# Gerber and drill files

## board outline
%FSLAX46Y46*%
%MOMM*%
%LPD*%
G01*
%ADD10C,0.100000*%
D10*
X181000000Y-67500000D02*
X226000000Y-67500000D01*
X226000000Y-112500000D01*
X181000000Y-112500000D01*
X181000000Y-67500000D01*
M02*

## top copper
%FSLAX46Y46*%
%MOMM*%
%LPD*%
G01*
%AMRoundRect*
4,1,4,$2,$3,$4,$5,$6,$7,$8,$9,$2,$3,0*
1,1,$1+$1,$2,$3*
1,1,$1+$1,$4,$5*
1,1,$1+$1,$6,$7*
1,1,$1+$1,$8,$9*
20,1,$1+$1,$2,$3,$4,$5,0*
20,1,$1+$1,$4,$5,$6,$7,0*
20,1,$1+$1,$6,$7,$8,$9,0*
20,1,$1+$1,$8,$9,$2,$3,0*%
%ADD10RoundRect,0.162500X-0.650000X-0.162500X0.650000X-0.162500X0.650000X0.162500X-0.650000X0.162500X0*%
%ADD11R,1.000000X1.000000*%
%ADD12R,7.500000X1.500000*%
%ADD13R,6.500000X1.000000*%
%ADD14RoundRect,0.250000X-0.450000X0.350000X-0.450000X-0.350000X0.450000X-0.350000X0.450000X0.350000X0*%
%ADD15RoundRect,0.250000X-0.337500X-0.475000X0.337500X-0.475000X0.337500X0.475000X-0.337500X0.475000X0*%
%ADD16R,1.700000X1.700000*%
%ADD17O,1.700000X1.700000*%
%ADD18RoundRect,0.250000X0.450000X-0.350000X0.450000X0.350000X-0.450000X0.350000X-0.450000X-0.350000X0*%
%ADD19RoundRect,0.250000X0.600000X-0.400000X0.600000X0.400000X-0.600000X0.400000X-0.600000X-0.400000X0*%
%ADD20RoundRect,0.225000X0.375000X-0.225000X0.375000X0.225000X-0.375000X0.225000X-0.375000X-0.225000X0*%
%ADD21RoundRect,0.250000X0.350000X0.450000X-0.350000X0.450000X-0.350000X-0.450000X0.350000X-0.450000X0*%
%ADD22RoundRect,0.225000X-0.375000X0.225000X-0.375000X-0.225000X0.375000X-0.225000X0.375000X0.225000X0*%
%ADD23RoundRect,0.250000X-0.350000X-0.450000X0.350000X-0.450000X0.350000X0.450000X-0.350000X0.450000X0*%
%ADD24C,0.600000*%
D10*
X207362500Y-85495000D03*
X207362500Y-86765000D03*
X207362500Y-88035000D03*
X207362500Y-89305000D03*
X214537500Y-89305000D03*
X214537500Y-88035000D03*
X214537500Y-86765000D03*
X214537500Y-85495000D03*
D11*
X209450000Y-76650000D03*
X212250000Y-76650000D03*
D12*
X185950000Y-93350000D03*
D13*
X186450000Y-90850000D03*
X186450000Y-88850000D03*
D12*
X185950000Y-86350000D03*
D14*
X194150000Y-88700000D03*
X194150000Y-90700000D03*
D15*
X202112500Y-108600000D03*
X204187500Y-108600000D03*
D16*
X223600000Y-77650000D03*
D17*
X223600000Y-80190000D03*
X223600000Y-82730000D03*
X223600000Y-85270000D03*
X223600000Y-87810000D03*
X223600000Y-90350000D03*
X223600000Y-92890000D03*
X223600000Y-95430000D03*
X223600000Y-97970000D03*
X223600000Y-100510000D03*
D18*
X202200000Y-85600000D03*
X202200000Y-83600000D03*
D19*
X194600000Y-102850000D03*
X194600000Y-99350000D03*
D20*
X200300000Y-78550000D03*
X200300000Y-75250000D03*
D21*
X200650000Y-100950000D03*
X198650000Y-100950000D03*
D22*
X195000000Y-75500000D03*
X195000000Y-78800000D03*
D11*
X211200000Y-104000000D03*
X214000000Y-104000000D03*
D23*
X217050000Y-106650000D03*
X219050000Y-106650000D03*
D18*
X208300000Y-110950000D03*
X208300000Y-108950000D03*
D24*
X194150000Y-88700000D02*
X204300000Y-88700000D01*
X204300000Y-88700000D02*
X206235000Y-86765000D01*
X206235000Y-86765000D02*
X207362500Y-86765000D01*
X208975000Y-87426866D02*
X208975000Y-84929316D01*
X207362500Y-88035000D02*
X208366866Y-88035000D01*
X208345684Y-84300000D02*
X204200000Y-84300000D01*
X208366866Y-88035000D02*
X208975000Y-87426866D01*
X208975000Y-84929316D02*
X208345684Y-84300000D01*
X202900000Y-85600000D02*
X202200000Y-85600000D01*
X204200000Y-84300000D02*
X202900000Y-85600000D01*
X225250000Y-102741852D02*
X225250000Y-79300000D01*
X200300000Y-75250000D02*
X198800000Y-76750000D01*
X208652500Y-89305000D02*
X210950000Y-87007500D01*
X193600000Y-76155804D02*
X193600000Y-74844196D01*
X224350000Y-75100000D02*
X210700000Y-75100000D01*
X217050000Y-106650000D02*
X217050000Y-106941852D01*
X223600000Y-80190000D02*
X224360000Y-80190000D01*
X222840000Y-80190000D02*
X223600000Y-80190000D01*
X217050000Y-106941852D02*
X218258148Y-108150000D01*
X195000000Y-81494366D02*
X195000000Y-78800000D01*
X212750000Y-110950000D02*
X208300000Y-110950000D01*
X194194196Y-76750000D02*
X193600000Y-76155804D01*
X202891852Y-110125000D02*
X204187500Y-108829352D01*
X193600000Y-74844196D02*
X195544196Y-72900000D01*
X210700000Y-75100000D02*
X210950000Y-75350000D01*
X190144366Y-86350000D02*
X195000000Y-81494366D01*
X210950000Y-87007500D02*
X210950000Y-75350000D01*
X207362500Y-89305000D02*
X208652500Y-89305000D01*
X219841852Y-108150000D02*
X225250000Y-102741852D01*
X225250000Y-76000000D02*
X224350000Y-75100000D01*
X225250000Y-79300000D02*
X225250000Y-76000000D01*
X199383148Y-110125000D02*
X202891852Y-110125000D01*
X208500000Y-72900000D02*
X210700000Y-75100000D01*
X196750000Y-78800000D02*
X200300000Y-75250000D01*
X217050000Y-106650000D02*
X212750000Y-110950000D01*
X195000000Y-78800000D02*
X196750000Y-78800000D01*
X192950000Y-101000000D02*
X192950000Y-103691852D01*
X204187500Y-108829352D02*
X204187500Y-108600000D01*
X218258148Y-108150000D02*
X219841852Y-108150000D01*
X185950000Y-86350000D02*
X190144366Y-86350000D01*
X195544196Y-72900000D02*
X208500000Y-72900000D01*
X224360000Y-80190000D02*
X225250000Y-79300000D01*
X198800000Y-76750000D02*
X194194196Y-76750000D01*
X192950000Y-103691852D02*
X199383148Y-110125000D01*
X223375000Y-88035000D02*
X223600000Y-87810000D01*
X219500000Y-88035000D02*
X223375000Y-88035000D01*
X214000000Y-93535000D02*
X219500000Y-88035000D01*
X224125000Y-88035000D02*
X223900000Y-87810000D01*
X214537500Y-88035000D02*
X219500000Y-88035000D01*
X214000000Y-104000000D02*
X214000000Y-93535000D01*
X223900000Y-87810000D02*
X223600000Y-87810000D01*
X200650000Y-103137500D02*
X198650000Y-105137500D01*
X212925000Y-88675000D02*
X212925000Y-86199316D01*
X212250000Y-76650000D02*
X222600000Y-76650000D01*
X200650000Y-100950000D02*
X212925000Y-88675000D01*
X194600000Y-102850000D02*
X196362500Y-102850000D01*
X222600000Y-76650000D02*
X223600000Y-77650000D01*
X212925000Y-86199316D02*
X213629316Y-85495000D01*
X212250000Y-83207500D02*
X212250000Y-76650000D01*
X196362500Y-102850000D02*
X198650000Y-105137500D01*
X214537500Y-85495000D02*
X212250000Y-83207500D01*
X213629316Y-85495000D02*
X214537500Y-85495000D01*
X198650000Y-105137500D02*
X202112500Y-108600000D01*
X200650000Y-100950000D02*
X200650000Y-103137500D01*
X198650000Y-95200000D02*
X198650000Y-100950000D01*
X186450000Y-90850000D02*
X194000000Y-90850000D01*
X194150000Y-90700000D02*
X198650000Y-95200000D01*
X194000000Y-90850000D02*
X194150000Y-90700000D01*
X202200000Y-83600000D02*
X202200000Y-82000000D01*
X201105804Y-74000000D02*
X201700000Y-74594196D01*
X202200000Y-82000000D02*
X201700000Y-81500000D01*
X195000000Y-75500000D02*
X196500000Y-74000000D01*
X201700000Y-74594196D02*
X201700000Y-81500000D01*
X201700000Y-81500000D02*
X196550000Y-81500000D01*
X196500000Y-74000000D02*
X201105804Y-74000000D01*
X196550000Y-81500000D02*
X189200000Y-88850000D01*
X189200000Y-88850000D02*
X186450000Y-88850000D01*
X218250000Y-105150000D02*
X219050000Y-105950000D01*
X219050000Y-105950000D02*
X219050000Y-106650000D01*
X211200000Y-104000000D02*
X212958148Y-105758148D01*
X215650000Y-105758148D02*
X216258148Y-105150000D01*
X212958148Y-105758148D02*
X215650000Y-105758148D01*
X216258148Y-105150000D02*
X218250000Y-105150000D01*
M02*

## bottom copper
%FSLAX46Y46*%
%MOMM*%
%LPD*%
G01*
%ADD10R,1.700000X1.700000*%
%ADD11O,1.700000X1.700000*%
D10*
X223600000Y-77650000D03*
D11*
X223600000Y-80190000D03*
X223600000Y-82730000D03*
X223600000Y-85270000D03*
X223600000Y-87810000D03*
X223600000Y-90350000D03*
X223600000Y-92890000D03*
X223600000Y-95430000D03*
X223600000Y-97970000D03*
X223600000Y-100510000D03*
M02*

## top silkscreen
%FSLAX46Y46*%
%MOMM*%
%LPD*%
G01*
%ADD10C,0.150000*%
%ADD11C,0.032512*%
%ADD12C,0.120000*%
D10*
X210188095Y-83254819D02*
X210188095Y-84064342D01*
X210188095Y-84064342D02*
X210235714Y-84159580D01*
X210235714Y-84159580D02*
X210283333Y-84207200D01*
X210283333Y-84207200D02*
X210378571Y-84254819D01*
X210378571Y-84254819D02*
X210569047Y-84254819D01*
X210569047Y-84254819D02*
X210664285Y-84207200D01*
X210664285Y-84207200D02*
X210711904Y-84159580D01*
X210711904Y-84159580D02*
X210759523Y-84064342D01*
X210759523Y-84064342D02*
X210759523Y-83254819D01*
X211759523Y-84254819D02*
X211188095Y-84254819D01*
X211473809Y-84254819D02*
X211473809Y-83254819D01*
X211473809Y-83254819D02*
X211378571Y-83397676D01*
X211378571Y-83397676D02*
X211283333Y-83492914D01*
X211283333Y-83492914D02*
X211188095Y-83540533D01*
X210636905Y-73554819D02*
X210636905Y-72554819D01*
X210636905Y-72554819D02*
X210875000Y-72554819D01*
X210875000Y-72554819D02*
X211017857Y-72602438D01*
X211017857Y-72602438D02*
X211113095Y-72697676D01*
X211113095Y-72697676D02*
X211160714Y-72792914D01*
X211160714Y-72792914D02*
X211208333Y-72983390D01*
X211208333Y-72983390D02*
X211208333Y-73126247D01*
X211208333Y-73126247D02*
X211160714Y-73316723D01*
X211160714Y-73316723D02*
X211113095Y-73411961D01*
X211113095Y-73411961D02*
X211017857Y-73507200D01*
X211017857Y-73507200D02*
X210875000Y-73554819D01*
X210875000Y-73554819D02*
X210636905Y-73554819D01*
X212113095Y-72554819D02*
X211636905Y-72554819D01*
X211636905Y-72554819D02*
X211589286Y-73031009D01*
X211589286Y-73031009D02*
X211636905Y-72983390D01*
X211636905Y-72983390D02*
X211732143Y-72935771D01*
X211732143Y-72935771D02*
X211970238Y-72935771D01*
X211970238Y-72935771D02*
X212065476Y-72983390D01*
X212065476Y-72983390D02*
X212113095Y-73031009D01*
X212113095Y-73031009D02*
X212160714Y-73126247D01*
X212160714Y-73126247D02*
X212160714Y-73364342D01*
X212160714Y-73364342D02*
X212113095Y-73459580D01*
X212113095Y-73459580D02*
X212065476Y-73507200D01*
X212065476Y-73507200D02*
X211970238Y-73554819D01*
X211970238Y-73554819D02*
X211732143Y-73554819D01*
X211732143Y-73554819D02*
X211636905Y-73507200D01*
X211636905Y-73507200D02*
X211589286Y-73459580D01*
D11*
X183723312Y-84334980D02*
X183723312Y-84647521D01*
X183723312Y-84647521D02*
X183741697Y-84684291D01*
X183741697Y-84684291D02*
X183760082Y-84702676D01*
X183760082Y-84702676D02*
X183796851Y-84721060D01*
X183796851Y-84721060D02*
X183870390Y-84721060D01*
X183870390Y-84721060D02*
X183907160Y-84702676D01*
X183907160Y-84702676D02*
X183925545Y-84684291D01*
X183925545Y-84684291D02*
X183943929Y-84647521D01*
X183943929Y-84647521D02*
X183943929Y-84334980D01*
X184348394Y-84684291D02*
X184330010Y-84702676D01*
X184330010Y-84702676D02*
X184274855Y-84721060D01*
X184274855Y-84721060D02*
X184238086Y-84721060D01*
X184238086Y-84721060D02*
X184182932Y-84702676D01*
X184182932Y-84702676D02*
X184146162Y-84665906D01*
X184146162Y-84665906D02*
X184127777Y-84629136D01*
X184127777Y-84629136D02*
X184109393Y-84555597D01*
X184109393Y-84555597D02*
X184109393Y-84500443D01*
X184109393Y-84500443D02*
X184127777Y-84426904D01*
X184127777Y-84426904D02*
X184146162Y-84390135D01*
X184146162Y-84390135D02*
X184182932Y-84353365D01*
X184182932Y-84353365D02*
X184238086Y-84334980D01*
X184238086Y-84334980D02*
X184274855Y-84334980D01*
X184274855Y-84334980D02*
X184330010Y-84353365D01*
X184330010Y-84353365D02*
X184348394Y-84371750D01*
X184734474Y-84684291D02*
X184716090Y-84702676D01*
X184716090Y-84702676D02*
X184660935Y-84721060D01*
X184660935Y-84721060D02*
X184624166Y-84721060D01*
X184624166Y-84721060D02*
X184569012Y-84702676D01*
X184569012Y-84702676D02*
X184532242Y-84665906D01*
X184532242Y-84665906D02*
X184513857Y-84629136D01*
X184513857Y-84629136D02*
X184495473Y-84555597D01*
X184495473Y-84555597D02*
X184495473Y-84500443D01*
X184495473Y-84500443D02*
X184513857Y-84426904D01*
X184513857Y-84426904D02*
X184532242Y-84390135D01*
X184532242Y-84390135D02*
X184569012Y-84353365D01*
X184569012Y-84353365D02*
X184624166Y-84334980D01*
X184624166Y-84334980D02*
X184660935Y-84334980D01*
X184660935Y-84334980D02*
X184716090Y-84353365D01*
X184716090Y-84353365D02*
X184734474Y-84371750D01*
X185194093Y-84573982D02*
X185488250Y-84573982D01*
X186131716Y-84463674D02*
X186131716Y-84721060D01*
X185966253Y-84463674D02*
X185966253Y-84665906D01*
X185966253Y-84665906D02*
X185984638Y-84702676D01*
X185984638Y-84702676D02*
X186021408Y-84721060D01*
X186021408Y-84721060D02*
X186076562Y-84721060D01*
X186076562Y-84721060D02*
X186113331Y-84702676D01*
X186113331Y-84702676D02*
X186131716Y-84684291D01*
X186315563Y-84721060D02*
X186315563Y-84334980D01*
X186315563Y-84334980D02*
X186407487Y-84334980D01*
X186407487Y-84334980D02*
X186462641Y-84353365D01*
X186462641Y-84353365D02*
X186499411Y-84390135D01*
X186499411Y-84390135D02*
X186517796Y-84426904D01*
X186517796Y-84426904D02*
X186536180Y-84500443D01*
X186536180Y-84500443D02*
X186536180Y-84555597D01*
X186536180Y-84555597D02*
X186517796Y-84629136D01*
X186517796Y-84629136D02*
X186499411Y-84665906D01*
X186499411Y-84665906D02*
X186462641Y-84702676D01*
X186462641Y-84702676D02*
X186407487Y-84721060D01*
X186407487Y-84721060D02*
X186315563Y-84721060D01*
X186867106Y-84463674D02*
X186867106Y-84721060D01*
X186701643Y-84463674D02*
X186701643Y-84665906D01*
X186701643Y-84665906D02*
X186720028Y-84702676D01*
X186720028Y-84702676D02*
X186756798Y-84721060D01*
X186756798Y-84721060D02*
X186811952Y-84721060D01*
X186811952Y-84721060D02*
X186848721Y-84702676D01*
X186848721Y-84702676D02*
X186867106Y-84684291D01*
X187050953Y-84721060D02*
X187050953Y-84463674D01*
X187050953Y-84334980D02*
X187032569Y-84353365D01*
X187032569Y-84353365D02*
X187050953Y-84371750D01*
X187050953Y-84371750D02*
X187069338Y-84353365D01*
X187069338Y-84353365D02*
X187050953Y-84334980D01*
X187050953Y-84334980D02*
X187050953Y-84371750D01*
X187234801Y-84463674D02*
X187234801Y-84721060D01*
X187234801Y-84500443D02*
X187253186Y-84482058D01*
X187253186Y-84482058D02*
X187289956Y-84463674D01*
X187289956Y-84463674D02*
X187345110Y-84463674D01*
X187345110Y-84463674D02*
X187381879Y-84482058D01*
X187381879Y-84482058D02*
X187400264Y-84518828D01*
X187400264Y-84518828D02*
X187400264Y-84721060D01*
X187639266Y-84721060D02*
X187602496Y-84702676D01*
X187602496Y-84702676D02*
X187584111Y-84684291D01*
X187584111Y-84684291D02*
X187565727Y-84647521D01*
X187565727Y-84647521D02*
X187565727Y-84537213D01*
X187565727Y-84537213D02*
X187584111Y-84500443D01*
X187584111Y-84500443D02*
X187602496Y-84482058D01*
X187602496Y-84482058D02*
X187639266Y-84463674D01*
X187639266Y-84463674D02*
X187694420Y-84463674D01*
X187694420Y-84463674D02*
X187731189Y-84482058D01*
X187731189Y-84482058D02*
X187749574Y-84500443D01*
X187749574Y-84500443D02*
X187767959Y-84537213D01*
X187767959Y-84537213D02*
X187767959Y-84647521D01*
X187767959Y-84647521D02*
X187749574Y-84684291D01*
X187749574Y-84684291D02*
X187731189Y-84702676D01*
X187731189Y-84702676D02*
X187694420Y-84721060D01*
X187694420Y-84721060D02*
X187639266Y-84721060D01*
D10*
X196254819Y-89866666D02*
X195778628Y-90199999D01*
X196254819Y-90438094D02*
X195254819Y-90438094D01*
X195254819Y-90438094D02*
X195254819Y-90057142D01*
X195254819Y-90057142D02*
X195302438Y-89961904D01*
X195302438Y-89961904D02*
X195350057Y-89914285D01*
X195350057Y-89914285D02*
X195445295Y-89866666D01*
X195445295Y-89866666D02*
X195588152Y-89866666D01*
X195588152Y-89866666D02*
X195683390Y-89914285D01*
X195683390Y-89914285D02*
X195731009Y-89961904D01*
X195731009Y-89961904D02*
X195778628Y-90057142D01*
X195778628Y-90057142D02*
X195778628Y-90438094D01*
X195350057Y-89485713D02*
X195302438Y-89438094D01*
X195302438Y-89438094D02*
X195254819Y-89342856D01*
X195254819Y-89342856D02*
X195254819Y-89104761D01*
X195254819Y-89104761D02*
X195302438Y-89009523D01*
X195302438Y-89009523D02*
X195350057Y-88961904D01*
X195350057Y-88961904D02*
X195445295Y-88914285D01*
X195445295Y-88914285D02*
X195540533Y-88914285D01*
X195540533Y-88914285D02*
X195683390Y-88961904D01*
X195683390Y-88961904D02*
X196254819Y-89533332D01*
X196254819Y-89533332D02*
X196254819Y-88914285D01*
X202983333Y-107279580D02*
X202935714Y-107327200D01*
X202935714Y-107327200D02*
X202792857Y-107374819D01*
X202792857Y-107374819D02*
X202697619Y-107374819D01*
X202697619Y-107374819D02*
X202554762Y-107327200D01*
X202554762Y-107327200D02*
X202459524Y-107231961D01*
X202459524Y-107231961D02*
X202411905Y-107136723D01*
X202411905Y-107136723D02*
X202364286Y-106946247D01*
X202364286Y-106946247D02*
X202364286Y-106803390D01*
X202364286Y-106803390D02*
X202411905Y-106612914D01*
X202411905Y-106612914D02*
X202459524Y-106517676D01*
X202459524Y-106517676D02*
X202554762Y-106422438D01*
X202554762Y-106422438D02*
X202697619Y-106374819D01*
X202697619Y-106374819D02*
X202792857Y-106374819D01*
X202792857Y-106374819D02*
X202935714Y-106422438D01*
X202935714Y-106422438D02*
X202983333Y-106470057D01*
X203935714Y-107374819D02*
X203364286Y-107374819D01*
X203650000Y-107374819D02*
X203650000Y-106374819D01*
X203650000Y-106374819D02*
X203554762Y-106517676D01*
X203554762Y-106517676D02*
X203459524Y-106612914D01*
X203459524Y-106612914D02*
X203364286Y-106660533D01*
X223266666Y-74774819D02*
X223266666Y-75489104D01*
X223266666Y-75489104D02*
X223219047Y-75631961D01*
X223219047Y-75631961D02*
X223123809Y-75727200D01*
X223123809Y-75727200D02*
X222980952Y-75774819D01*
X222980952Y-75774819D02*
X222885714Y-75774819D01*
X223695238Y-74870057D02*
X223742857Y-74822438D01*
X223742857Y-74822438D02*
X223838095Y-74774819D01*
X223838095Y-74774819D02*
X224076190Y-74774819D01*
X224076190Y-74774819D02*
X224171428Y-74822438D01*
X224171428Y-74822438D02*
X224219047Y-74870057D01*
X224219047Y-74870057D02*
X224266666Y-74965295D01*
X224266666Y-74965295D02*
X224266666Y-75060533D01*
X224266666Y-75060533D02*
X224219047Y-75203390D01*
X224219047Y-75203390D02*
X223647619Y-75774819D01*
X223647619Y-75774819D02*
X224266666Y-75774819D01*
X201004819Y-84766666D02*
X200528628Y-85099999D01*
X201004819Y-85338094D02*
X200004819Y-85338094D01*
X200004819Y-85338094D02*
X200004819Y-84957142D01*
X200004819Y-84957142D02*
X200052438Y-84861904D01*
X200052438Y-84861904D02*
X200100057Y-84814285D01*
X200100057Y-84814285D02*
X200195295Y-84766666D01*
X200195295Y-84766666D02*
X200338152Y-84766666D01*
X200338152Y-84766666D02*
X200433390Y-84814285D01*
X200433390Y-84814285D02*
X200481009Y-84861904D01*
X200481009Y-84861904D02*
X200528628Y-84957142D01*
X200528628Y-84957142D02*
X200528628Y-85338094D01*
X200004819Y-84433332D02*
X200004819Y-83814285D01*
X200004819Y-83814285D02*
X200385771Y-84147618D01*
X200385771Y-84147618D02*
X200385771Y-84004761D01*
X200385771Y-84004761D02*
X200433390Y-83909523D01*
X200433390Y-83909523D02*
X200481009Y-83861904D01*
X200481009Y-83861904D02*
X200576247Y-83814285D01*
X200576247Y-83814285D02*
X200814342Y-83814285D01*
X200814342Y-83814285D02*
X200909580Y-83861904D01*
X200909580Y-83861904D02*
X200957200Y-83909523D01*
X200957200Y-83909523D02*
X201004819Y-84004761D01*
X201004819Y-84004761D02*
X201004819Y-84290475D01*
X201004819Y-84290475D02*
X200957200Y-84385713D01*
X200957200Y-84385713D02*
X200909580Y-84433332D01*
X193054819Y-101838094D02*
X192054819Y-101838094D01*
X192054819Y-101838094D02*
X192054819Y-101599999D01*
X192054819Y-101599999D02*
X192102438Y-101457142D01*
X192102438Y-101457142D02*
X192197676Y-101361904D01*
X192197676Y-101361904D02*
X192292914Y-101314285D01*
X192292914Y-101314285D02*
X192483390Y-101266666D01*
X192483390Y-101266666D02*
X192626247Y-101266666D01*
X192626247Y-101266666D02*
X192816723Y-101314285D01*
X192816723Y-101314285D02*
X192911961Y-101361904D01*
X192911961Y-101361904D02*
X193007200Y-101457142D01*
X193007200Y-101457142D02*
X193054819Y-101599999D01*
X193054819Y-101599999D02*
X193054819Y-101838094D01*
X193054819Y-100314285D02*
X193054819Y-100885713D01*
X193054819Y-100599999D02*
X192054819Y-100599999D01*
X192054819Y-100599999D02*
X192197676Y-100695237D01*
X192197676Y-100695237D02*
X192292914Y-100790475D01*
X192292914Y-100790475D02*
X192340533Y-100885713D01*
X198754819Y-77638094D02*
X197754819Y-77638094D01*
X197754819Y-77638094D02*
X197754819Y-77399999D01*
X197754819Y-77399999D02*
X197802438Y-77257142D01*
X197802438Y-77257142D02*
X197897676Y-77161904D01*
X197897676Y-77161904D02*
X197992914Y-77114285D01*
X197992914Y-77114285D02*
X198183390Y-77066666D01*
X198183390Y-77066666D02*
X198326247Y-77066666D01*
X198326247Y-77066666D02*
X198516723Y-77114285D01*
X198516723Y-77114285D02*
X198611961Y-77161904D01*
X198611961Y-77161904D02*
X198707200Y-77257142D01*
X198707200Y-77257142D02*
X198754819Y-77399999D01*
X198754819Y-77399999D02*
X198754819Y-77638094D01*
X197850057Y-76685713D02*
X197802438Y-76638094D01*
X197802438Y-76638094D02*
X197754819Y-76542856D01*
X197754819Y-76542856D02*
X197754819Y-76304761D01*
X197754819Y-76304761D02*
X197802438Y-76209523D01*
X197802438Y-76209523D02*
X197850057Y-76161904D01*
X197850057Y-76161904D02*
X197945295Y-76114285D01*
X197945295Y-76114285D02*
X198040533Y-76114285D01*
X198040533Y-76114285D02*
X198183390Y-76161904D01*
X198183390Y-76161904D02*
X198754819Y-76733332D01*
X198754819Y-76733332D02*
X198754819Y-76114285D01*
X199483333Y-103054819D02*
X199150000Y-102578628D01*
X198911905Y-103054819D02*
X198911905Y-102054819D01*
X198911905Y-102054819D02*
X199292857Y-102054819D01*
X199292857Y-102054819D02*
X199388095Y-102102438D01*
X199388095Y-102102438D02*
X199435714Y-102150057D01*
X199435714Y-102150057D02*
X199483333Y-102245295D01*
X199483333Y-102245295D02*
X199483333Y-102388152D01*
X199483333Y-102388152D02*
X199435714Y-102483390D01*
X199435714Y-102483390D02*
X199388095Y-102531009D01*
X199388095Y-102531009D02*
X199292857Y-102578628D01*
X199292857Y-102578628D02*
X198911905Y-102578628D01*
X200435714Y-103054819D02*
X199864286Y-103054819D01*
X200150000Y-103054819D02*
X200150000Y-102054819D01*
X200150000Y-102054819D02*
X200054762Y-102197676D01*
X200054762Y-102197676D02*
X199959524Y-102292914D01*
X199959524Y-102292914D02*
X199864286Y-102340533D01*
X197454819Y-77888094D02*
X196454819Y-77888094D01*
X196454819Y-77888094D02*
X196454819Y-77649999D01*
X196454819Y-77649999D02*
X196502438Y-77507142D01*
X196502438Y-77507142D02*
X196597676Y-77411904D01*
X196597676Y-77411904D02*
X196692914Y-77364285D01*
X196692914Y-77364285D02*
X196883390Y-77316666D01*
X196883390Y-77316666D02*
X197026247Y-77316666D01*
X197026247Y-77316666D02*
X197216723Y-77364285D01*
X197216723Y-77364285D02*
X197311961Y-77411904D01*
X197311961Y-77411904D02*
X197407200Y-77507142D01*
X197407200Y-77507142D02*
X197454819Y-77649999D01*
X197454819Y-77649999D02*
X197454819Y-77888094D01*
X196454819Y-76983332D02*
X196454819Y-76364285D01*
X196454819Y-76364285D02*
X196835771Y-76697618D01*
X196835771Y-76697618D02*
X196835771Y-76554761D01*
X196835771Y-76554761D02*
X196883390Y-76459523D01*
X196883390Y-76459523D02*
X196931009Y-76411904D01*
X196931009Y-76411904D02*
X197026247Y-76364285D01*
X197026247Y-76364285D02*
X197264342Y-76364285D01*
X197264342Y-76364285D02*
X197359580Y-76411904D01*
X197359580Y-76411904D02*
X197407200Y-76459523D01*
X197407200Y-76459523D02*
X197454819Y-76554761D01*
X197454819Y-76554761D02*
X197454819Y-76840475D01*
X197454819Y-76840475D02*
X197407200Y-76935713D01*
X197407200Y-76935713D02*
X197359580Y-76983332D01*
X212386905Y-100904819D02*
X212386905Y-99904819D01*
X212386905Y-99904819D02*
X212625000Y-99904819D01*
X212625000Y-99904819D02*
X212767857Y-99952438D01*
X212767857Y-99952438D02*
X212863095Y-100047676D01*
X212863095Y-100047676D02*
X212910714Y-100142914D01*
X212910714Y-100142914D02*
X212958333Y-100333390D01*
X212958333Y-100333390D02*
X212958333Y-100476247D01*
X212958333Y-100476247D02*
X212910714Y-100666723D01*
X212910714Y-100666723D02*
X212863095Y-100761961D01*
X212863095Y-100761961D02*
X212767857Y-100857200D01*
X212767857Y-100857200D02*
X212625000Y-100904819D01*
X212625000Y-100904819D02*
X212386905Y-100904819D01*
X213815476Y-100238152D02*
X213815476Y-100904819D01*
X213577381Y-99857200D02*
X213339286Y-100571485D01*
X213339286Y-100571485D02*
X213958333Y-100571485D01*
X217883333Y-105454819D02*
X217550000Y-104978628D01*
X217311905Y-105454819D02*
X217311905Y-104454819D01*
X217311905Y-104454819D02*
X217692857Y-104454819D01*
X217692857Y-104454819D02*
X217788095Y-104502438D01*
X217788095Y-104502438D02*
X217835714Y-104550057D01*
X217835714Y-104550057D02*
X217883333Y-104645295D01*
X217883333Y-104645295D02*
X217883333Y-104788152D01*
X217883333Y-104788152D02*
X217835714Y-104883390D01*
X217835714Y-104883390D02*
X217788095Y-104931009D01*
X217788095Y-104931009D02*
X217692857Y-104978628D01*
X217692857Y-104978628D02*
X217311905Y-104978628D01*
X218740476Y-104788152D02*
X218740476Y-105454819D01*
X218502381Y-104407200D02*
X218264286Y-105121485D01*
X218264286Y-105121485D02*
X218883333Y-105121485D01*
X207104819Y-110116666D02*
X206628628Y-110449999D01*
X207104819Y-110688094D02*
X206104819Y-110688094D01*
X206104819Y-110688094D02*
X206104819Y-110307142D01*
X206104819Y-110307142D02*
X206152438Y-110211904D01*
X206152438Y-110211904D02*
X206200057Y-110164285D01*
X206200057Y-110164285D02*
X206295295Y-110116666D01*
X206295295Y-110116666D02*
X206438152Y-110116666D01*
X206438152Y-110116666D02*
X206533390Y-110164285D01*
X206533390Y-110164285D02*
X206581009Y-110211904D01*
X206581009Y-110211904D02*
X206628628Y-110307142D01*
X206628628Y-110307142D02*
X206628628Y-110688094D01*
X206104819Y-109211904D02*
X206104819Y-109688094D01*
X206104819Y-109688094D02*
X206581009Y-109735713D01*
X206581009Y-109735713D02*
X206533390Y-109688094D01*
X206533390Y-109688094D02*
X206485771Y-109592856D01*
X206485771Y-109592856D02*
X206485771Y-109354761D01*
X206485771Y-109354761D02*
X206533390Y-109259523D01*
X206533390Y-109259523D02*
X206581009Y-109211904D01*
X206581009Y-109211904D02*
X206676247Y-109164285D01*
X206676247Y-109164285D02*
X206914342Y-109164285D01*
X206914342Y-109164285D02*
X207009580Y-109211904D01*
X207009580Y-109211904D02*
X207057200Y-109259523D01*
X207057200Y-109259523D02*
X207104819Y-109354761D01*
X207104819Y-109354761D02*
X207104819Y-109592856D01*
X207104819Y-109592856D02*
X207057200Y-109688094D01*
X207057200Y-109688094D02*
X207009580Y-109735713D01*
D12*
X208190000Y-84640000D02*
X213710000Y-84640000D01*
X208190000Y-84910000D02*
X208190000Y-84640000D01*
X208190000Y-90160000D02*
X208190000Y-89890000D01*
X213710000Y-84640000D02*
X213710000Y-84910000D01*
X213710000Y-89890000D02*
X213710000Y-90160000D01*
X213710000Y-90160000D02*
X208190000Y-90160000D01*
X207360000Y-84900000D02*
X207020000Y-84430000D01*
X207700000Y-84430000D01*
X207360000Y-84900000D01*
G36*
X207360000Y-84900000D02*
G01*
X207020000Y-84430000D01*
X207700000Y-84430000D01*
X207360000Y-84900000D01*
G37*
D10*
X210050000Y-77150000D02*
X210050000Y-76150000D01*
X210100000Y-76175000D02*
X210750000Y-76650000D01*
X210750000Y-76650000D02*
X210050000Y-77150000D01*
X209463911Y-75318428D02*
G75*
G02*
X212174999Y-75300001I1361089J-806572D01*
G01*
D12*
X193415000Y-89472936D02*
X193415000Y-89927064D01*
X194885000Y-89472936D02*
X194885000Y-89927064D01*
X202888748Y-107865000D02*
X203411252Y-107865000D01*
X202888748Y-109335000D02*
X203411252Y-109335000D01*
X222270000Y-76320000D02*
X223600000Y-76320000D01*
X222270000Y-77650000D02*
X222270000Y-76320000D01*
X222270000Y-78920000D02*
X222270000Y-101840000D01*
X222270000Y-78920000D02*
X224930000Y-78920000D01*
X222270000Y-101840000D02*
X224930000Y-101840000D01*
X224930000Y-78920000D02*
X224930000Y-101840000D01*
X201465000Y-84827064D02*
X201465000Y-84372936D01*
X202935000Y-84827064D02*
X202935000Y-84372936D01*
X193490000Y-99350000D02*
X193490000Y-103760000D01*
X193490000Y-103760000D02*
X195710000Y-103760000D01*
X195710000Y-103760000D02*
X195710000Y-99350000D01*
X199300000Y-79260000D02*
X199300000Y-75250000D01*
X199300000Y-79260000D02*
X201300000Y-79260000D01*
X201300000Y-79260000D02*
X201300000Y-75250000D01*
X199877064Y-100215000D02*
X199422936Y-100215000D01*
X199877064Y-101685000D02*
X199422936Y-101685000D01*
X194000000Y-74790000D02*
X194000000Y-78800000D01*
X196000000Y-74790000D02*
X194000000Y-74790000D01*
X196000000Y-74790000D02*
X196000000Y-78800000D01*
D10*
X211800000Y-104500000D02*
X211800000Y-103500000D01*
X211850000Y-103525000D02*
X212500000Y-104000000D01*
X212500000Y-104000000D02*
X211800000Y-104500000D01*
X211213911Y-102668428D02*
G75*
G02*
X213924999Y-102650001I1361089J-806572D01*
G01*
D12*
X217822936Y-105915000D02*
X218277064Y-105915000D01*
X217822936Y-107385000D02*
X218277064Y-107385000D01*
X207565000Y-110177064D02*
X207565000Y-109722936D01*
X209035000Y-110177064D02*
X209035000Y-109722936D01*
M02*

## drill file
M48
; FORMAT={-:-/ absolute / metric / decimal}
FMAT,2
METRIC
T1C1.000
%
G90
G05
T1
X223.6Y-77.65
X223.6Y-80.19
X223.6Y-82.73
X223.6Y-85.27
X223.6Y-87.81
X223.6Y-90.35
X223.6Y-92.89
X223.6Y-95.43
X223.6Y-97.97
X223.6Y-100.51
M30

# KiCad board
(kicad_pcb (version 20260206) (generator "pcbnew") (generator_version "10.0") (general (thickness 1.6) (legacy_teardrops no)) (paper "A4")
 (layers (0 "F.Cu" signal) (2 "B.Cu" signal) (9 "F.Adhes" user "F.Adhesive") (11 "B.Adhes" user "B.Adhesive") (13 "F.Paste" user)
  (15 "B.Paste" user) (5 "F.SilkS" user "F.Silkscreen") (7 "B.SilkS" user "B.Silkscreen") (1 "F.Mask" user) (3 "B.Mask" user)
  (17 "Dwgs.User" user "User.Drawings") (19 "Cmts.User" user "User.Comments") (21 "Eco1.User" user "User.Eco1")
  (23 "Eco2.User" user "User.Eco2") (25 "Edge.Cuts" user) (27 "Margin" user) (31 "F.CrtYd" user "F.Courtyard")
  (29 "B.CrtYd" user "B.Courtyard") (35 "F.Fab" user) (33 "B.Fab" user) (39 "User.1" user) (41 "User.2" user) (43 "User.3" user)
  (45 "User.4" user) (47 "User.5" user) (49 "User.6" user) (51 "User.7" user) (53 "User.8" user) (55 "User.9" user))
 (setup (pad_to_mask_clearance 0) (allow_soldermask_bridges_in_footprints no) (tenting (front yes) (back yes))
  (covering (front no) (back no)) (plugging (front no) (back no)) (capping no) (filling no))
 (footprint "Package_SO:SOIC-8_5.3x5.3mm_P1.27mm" (layer "F.Cu") (at 210.95 87.4)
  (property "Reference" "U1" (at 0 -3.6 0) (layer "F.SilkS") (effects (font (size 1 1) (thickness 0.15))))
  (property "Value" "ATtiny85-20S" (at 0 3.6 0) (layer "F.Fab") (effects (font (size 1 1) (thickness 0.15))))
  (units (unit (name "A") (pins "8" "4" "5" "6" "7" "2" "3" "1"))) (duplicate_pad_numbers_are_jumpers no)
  (fp_line (start -2.76 -2.76) (end 2.76 -2.76) (stroke (width 0.12) (type solid)) (layer "F.SilkS"))
  (fp_line (start -2.76 -2.49) (end -2.76 -2.76) (stroke (width 0.12) (type solid)) (layer "F.SilkS"))
  (fp_line (start -2.76 2.76) (end -2.76 2.49) (stroke (width 0.12) (type solid)) (layer "F.SilkS"))
  (fp_line (start 2.76 -2.76) (end 2.76 -2.49) (stroke (width 0.12) (type solid)) (layer "F.SilkS"))
  (fp_line (start 2.76 2.49) (end 2.76 2.76) (stroke (width 0.12) (type solid)) (layer "F.SilkS"))
  (fp_line (start 2.76 2.76) (end -2.76 2.76) (stroke (width 0.12) (type solid)) (layer "F.SilkS"))
  (fp_poly (pts (xy -3.59 -2.5) (xy -3.93 -2.97) (xy -3.25 -2.97)) (stroke (width 0.12) (type solid)) (fill yes) (layer "F.SilkS"))
  (pad "1" smd roundrect (at -3.5875 -1.905) (size 1.625 0.65) (layers "F.Cu" "F.Mask" "F.Paste") (roundrect_rratio 0.25)
   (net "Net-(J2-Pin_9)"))
  (pad "2" smd roundrect (at -3.5875 -0.635) (size 1.625 0.65) (layers "F.Cu" "F.Mask" "F.Paste") (roundrect_rratio 0.25)
   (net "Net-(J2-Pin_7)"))
  (pad "3" smd roundrect (at -3.5875 0.635) (size 1.625 0.65) (layers "F.Cu" "F.Mask" "F.Paste") (roundrect_rratio 0.25)
   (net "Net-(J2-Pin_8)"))
  (pad "4" smd roundrect (at -3.5875 1.905) (size 1.625 0.65) (layers "F.Cu" "F.Mask" "F.Paste") (roundrect_rratio 0.25) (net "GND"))
  (pad "5" smd roundrect (at 3.5875 1.905) (size 1.625 0.65) (layers "F.Cu" "F.Mask" "F.Paste") (roundrect_rratio 0.25)
   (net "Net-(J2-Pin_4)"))
  (pad "6" smd roundrect (at 3.5875 0.635) (size 1.625 0.65) (layers "F.Cu" "F.Mask" "F.Paste") (roundrect_rratio 0.25) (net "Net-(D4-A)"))
  (pad "7" smd roundrect (at 3.5875 -0.635) (size 1.625 0.65) (layers "F.Cu" "F.Mask" "F.Paste") (roundrect_rratio 0.25)
   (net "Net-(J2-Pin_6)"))
  (pad "8" smd roundrect (at 3.5875 -1.905) (size 1.625 0.65) (layers "F.Cu" "F.Mask" "F.Paste") (roundrect_rratio 0.25) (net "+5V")))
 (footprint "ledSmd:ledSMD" (layer "F.Cu") (at 211.25 76.65)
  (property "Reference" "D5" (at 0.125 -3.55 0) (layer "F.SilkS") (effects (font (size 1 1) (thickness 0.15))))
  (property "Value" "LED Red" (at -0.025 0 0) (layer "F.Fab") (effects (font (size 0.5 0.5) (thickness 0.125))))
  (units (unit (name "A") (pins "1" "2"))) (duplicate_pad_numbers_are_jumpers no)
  (fp_line (start -1.2 0.5) (end -1.2 -0.5) (stroke (width 0.15) (type solid)) (layer "F.SilkS"))
  (fp_line (start -1.15 -0.475) (end -0.5 0) (stroke (width 0.15) (type solid)) (layer "F.SilkS"))
  (fp_line (start -0.5 0) (end -1.2 0.5) (stroke (width 0.15) (type solid)) (layer "F.SilkS"))
  (fp_arc (start -1.786089 -1.331572) (mid -0.435753 -2.107089) (end 0.924999 -1.349999) (stroke (width 0.15) (type solid))
   (layer "F.SilkS"))
  (pad "1" smd rect (at -1.8 0) (size 1 1) (layers "F.Cu" "F.Mask" "F.Paste") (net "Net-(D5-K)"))
  (pad "2" smd rect (at 1 0) (size 1 1) (layers "F.Cu" "F.Mask" "F.Paste") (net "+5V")))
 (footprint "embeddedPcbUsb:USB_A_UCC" (layer "F.Cu") (at 186.15 89.85)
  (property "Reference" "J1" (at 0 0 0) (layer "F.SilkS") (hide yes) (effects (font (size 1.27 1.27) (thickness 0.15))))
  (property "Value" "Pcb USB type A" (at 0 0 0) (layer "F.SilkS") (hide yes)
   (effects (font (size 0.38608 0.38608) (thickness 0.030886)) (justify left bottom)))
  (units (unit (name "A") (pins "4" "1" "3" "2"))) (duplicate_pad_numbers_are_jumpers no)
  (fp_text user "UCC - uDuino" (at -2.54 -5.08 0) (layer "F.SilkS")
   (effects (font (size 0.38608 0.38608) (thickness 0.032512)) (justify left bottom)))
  (pad "1" smd rect (at -0.2 3.5) (size 7.5 1.5) (layers "F.Cu" "F.Mask" "F.Paste") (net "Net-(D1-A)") (solder_mask_margin 0.1016))
  (pad "2" smd rect (at 0.3 1) (size 6.5 1) (layers "F.Cu" "F.Mask" "F.Paste") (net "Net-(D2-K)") (solder_mask_margin 0.1016))
  (pad "3" smd rect (at 0.3 -1) (size 6.5 1) (layers "F.Cu" "F.Mask" "F.Paste") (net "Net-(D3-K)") (solder_mask_margin 0.1016))
  (pad "4" smd rect (at -0.2 -3.5) (size 7.5 1.5) (layers "F.Cu" "F.Mask" "F.Paste") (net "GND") (solder_mask_margin 0.1016)))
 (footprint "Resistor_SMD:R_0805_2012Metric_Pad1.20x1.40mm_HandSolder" (layer "F.Cu") (at 194.15 89.7 -90)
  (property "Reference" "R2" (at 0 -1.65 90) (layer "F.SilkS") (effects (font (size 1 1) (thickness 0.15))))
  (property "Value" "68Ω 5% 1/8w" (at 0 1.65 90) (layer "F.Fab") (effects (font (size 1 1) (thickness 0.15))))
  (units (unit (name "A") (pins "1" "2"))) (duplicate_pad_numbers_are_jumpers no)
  (fp_line (start -0.227064 0.735) (end 0.227064 0.735) (stroke (width 0.12) (type solid)) (layer "F.SilkS"))
  (fp_line (start -0.227064 -0.735) (end 0.227064 -0.735) (stroke (width 0.12) (type solid)) (layer "F.SilkS"))
  (pad "1" smd roundrect (at -1 0 270) (size 1.2 1.4) (layers "F.Cu" "F.Mask" "F.Paste") (roundrect_rratio 0.208333) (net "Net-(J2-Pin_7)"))
  (pad "2" smd roundrect (at 1 0 270) (size 1.2 1.4) (layers "F.Cu" "F.Mask" "F.Paste") (roundrect_rratio 0.208333) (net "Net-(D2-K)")))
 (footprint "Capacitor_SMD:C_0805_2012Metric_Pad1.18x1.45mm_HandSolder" (layer "F.Cu") (at 203.15 108.6)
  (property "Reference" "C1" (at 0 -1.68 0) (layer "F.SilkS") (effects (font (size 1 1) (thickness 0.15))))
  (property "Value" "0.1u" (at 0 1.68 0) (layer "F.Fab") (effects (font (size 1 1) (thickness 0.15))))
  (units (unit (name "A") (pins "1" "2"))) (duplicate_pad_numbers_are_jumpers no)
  (fp_line (start -0.261252 -0.735) (end 0.261252 -0.735) (stroke (width 0.12) (type solid)) (layer "F.SilkS"))
  (fp_line (start -0.261252 0.735) (end 0.261252 0.735) (stroke (width 0.12) (type solid)) (layer "F.SilkS"))
  (pad "1" smd roundrect (at -1.0375 0) (size 1.175 1.45) (layers "F.Cu" "F.Mask" "F.Paste") (roundrect_rratio 0.212766) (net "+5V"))
  (pad "2" smd roundrect (at 1.0375 0) (size 1.175 1.45) (layers "F.Cu" "F.Mask" "F.Paste") (roundrect_rratio 0.212766) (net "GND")))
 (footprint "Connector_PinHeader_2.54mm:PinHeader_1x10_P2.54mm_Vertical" (layer "F.Cu") (at 223.6 77.65)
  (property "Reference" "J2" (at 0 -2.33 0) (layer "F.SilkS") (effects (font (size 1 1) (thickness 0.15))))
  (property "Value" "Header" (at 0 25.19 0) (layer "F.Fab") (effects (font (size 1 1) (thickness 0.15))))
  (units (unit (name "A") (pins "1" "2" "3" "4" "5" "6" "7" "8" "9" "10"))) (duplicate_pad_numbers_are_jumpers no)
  (fp_line (start -1.33 -1.33) (end 0 -1.33) (stroke (width 0.12) (type solid)) (layer "F.SilkS"))
  (fp_line (start -1.33 0) (end -1.33 -1.33) (stroke (width 0.12) (type solid)) (layer "F.SilkS"))
  (fp_line (start -1.33 1.27) (end -1.33 24.19) (stroke (width 0.12) (type solid)) (layer "F.SilkS"))
  (fp_line (start -1.33 1.27) (end 1.33 1.27) (stroke (width 0.12) (type solid)) (layer "F.SilkS"))
  (fp_line (start -1.33 24.19) (end 1.33 24.19) (stroke (width 0.12) (type solid)) (layer "F.SilkS"))
  (fp_line (start 1.33 1.27) (end 1.33 24.19) (stroke (width 0.12) (type solid)) (layer "F.SilkS"))
  (pad "1" thru_hole rect (at 0 0) (size 1.7 1.7) (drill 1) (layers "*.Cu" "*.Mask") (remove_unused_layers no) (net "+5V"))
  (pad "2" thru_hole oval (at 0 2.54) (size 1.7 1.7) (drill 1) (layers "*.Cu" "*.Mask") (remove_unused_layers no) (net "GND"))
  (pad "3" thru_hole oval (at 0 5.08) (size 1.7 1.7) (drill 1) (layers "*.Cu" "*.Mask") (remove_unused_layers no)
   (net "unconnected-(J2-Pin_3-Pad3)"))
  (pad "4" thru_hole oval (at 0 7.62) (size 1.7 1.7) (drill 1) (layers "*.Cu" "*.Mask") (remove_unused_layers no) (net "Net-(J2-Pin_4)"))
  (pad "5" thru_hole oval (at 0 10.16) (size 1.7 1.7) (drill 1) (layers "*.Cu" "*.Mask") (remove_unused_layers no) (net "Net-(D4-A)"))
  (pad "6" thru_hole oval (at 0 12.7) (size 1.7 1.7) (drill 1) (layers "*.Cu" "*.Mask") (remove_unused_layers no) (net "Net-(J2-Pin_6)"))
  (pad "7" thru_hole oval (at 0 15.24) (size 1.7 1.7) (drill 1) (layers "*.Cu" "*.Mask") (remove_unused_layers no) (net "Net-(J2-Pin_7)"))
  (pad "8" thru_hole oval (at 0 17.78) (size 1.7 1.7) (drill 1) (layers "*.Cu" "*.Mask") (remove_unused_layers no) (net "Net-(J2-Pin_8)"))
  (pad "9" thru_hole oval (at 0 20.32) (size 1.7 1.7) (drill 1) (layers "*.Cu" "*.Mask") (remove_unused_layers no) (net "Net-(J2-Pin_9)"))
  (pad "10" thru_hole oval (at 0 22.86) (size 1.7 1.7) (drill 1) (layers "*.Cu" "*.Mask") (remove_unused_layers no)
   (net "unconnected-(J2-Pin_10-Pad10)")))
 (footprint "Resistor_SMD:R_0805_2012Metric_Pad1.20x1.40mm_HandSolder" (layer "F.Cu") (at 202.2 84.6 90)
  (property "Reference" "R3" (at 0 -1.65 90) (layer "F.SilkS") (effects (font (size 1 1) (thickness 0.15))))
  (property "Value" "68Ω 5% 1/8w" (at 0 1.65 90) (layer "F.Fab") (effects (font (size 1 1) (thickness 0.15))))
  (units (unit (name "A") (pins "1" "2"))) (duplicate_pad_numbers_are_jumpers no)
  (fp_line (start -0.227064 -0.735) (end 0.227064 -0.735) (stroke (width 0.12) (type solid)) (layer "F.SilkS"))
  (fp_line (start -0.227064 0.735) (end 0.227064 0.735) (stroke (width 0.12) (type solid)) (layer "F.SilkS"))
  (pad "1" smd roundrect (at -1 0 90) (size 1.2 1.4) (layers "F.Cu" "F.Mask" "F.Paste") (roundrect_rratio 0.208333) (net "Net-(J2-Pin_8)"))
  (pad "2" smd roundrect (at 1 0 90) (size 1.2 1.4) (layers "F.Cu" "F.Mask" "F.Paste") (roundrect_rratio 0.208333) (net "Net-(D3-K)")))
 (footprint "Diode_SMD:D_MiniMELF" (layer "F.Cu") (at 194.6 101.1 90)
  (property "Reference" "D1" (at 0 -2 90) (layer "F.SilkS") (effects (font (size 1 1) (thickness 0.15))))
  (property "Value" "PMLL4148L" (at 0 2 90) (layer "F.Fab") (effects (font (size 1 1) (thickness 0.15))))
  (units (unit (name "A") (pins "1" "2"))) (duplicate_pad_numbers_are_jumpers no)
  (fp_line (start 1.75 -1.11) (end -2.66 -1.11) (stroke (width 0.12) (type solid)) (layer "F.SilkS"))
  (fp_line (start -2.66 -1.11) (end -2.66 1.11) (stroke (width 0.12) (type solid)) (layer "F.SilkS"))
  (fp_line (start -2.66 1.11) (end 1.75 1.11) (stroke (width 0.12) (type solid)) (layer "F.SilkS"))
  (pad "1" smd roundrect (at -1.75 0 90) (size 1.3 1.7) (layers "F.Cu" "F.Mask" "F.Paste") (roundrect_rratio 0.1923076923) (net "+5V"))
  (pad "2" smd roundrect (at 1.75 0 90) (size 1.3 1.7) (layers "F.Cu" "F.Mask" "F.Paste") (roundrect_rratio 0.1923076923) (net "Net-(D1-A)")))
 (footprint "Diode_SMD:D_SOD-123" (layer "F.Cu") (at 200.3 76.9 90)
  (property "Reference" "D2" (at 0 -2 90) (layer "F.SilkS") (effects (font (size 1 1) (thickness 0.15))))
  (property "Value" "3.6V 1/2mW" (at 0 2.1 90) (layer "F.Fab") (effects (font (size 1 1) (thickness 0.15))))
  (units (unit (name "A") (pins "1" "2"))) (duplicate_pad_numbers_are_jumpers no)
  (fp_line (start -2.36 -1) (end 1.65 -1) (stroke (width 0.12) (type solid)) (layer "F.SilkS"))
  (fp_line (start -2.36 -1) (end -2.36 1) (stroke (width 0.12) (type solid)) (layer "F.SilkS"))
  (fp_line (start -2.36 1) (end 1.65 1) (stroke (width 0.12) (type solid)) (layer "F.SilkS"))
  (pad "1" smd roundrect (at -1.65 0 90) (size 0.9 1.2) (layers "F.Cu" "F.Mask" "F.Paste") (roundrect_rratio 0.25) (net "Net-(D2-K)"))
  (pad "2" smd roundrect (at 1.65 0 90) (size 0.9 1.2) (layers "F.Cu" "F.Mask" "F.Paste") (roundrect_rratio 0.25) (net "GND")))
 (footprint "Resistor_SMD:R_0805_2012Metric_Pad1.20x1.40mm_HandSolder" (layer "F.Cu") (at 199.65 100.95 180)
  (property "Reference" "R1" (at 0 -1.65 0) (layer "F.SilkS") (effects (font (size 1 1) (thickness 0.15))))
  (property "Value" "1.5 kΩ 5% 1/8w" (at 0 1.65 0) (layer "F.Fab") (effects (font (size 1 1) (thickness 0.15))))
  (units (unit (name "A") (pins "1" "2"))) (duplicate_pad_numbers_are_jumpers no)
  (fp_line (start -0.227064 0.735) (end 0.227064 0.735) (stroke (width 0.12) (type solid)) (layer "F.SilkS"))
  (fp_line (start -0.227064 -0.735) (end 0.227064 -0.735) (stroke (width 0.12) (type solid)) (layer "F.SilkS"))
  (pad "1" smd roundrect (at -1 0 180) (size 1.2 1.4) (layers "F.Cu" "F.Mask" "F.Paste") (roundrect_rratio 0.208333) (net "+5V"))
  (pad "2" smd roundrect (at 1 0 180) (size 1.2 1.4) (layers "F.Cu" "F.Mask" "F.Paste") (roundrect_rratio 0.208333) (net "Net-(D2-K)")))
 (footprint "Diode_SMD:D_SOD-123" (layer "F.Cu") (at 195 77.15 -90)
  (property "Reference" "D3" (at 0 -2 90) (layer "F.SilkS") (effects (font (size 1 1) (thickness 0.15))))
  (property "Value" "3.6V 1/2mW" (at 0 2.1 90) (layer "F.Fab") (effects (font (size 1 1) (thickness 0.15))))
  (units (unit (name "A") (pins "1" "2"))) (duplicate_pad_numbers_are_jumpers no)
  (fp_line (start -2.36 1) (end 1.65 1) (stroke (width 0.12) (type solid)) (layer "F.SilkS"))
  (fp_line (start -2.36 -1) (end -2.36 1) (stroke (width 0.12) (type solid)) (layer "F.SilkS"))
  (fp_line (start -2.36 -1) (end 1.65 -1) (stroke (width 0.12) (type solid)) (layer "F.SilkS"))
  (pad "1" smd roundrect (at -1.65 0 270) (size 0.9 1.2) (layers "F.Cu" "F.Mask" "F.Paste") (roundrect_rratio 0.25) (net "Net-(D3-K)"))
  (pad "2" smd roundrect (at 1.65 0 270) (size 0.9 1.2) (layers "F.Cu" "F.Mask" "F.Paste") (roundrect_rratio 0.25) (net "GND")))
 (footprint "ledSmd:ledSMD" (layer "F.Cu") (at 213 104)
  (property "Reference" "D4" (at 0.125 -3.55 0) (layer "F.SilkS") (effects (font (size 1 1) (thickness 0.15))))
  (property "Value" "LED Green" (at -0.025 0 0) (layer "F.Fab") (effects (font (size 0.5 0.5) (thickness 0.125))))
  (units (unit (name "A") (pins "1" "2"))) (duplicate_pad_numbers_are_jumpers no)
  (fp_line (start -1.2 0.5) (end -1.2 -0.5) (stroke (width 0.15) (type solid)) (layer "F.SilkS"))
  (fp_line (start -1.15 -0.475) (end -0.5 0) (stroke (width 0.15) (type solid)) (layer "F.SilkS"))
  (fp_line (start -0.5 0) (end -1.2 0.5) (stroke (width 0.15) (type solid)) (layer "F.SilkS"))
  (fp_arc (start -1.786089 -1.331572) (mid -0.435753 -2.107089) (end 0.924999 -1.349999) (stroke (width 0.15) (type solid))
   (layer "F.SilkS"))
  (pad "1" smd rect (at -1.8 0) (size 1 1) (layers "F.Cu" "F.Mask" "F.Paste") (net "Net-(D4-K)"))
  (pad "2" smd rect (at 1 0) (size 1 1) (layers "F.Cu" "F.Mask" "F.Paste") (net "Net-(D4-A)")))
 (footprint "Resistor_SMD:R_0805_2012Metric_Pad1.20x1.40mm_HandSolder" (layer "F.Cu") (at 218.05 106.65)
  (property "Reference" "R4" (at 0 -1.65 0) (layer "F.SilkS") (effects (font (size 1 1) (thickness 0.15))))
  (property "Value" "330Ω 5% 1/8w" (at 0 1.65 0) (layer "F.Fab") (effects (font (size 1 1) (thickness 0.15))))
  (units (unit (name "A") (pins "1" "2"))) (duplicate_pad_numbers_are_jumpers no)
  (fp_line (start -0.227064 -0.735) (end 0.227064 -0.735) (stroke (width 0.12) (type solid)) (layer "F.SilkS"))
  (fp_line (start -0.227064 0.735) (end 0.227064 0.735) (stroke (width 0.12) (type solid)) (layer "F.SilkS"))
  (pad "1" smd roundrect (at -1 0) (size 1.2 1.4) (layers "F.Cu" "F.Mask" "F.Paste") (roundrect_rratio 0.208333) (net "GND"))
  (pad "2" smd roundrect (at 1 0) (size 1.2 1.4) (layers "F.Cu" "F.Mask" "F.Paste") (roundrect_rratio 0.208333) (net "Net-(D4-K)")))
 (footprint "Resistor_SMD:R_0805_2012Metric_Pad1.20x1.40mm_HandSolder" (layer "F.Cu") (at 208.3 109.95 90)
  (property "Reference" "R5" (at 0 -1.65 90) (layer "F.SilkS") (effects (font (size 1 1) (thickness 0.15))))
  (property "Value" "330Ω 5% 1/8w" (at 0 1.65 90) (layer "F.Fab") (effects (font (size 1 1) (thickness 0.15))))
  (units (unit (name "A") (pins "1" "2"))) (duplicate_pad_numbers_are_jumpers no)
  (fp_line (start -0.227064 -0.735) (end 0.227064 -0.735) (stroke (width 0.12) (type solid)) (layer "F.SilkS"))
  (fp_line (start -0.227064 0.735) (end 0.227064 0.735) (stroke (width 0.12) (type solid)) (layer "F.SilkS"))
  (pad "1" smd roundrect (at -1 0 90) (size 1.2 1.4) (layers "F.Cu" "F.Mask" "F.Paste") (roundrect_rratio 0.208333) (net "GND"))
  (pad "2" smd roundrect (at 1 0 90) (size 1.2 1.4) (layers "F.Cu" "F.Mask" "F.Paste") (roundrect_rratio 0.208333) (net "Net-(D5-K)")))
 (gr_rect (start 181 67.5) (end 226 112.5) (stroke (width 0.1) (type default)) (fill no) (layer "Edge.Cuts"))
 (segment (start 194.15 88.7) (end 204.3 88.7) (width 0.6) (layer "F.Cu") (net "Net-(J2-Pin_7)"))
 (segment (start 204.3 88.7) (end 206.235 86.765) (width 0.6) (layer "F.Cu") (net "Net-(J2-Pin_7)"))
 (segment (start 206.235 86.765) (end 207.3625 86.765) (width 0.6) (layer "F.Cu") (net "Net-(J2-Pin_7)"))
 (segment (start 208.975 87.426866) (end 208.975 84.929316) (width 0.6) (layer "F.Cu") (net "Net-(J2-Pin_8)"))
 (segment (start 207.3625 88.035) (end 208.366866 88.035) (width 0.6) (layer "F.Cu") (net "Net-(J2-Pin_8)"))
 (segment (start 208.345684 84.3) (end 204.2 84.3) (width 0.6) (layer "F.Cu") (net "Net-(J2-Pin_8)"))
 (segment (start 208.366866 88.035) (end 208.975 87.426866) (width 0.6) (layer "F.Cu") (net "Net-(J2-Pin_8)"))
 (segment (start 208.975 84.929316) (end 208.345684 84.3) (width 0.6) (layer "F.Cu") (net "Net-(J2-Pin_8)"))
 (segment (start 202.9 85.6) (end 202.2 85.6) (width 0.6) (layer "F.Cu") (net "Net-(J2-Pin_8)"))
 (segment (start 204.2 84.3) (end 202.9 85.6) (width 0.6) (layer "F.Cu") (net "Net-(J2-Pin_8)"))
 (segment (start 225.25 102.741852) (end 225.25 79.3) (width 0.6) (layer "F.Cu") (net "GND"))
 (segment (start 200.3 75.25) (end 198.8 76.75) (width 0.6) (layer "F.Cu") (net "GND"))
 (segment (start 208.6525 89.305) (end 210.95 87.0075) (width 0.6) (layer "F.Cu") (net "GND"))
 (segment (start 193.6 76.155804) (end 193.6 74.844196) (width 0.6) (layer "F.Cu") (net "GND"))
 (segment (start 224.35 75.1) (end 210.7 75.1) (width 0.6) (layer "F.Cu") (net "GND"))
 (segment (start 217.05 106.65) (end 217.05 106.941852) (width 0.6) (layer "F.Cu") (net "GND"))
 (segment (start 223.6 80.19) (end 224.36 80.19) (width 0.6) (layer "F.Cu") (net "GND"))
 (segment (start 222.84 80.19) (end 223.6 80.19) (width 0.6) (layer "F.Cu") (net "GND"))
 (segment (start 217.05 106.941852) (end 218.258148 108.15) (width 0.6) (layer "F.Cu") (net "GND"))
 (segment (start 195 81.494366) (end 195 78.8) (width 0.6) (layer "F.Cu") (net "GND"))
 (segment (start 212.75 110.95) (end 208.3 110.95) (width 0.6) (layer "F.Cu") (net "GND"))
 (segment (start 194.194196 76.75) (end 193.6 76.155804) (width 0.6) (layer "F.Cu") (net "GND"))
 (segment (start 202.891852 110.125) (end 204.1875 108.829352) (width 0.6) (layer "F.Cu") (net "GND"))
 (segment (start 193.6 74.844196) (end 195.544196 72.9) (width 0.6) (layer "F.Cu") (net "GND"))
 (segment (start 210.7 75.1) (end 210.95 75.35) (width 0.6) (layer "F.Cu") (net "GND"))
 (segment (start 190.144366 86.35) (end 195 81.494366) (width 0.6) (layer "F.Cu") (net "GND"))
 (segment (start 210.95 87.0075) (end 210.95 75.35) (width 0.6) (layer "F.Cu") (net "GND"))
 (segment (start 207.3625 89.305) (end 208.6525 89.305) (width 0.6) (layer "F.Cu") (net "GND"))
 (segment (start 219.841852 108.15) (end 225.25 102.741852) (width 0.6) (layer "F.Cu") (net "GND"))
 (segment (start 225.25 76) (end 224.35 75.1) (width 0.6) (layer "F.Cu") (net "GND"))
 (segment (start 225.25 79.3) (end 225.25 76) (width 0.6) (layer "F.Cu") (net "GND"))
 (segment (start 199.383148 110.125) (end 202.891852 110.125) (width 0.6) (layer "F.Cu") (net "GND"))
 (segment (start 208.5 72.9) (end 210.7 75.1) (width 0.6) (layer "F.Cu") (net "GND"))
 (segment (start 196.75 78.8) (end 200.3 75.25) (width 0.6) (layer "F.Cu") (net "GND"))
 (segment (start 217.05 106.65) (end 212.75 110.95) (width 0.6) (layer "F.Cu") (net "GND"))
 (segment (start 195 78.8) (end 196.75 78.8) (width 0.6) (layer "F.Cu") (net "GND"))
 (segment (start 192.95 101) (end 192.95 103.691852) (width 0.6) (layer "F.Cu") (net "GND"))
 (segment (start 204.1875 108.829352) (end 204.1875 108.6) (width 0.6) (layer "F.Cu") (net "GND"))
 (segment (start 218.258148 108.15) (end 219.841852 108.15) (width 0.6) (layer "F.Cu") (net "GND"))
 (segment (start 185.95 86.35) (end 190.144366 86.35) (width 0.6) (layer "F.Cu") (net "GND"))
 (segment (start 195.544196 72.9) (end 208.5 72.9) (width 0.6) (layer "F.Cu") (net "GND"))
 (segment (start 224.36 80.19) (end 225.25 79.3) (width 0.6) (layer "F.Cu") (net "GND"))
 (segment (start 198.8 76.75) (end 194.194196 76.75) (width 0.6) (layer "F.Cu") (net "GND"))
 (segment (start 192.95 103.691852) (end 199.383148 110.125) (width 0.6) (layer "F.Cu") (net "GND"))
 (segment (start 223.375 88.035) (end 223.6 87.81) (width 0.6) (layer "F.Cu") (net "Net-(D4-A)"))
 (segment (start 219.5 88.035) (end 223.375 88.035) (width 0.6) (layer "F.Cu") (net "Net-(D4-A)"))
 (segment (start 214 93.535) (end 219.5 88.035) (width 0.6) (layer "F.Cu") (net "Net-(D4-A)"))
 (segment (start 224.125 88.035) (end 223.9 87.81) (width 0.6) (layer "F.Cu") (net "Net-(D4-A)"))
 (segment (start 214.5375 88.035) (end 219.5 88.035) (width 0.6) (layer "F.Cu") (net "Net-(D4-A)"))
 (segment (start 214 104) (end 214 93.535) (width 0.6) (layer "F.Cu") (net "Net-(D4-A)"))
 (segment (start 223.9 87.81) (end 223.6 87.81) (width 0.6) (layer "F.Cu") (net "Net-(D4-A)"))
 (segment (start 200.65 103.1375) (end 198.65 105.1375) (width 0.6) (layer "F.Cu") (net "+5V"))
 (segment (start 212.925 88.675) (end 212.925 86.199316) (width 0.6) (layer "F.Cu") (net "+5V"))
 (segment (start 212.25 76.65) (end 222.6 76.65) (width 0.6) (layer "F.Cu") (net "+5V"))
 (segment (start 200.65 100.95) (end 212.925 88.675) (width 0.6) (layer "F.Cu") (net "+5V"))
 (segment (start 194.6 102.85) (end 196.3625 102.85) (width 0.6) (layer "F.Cu") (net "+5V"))
 (segment (start 222.6 76.65) (end 223.6 77.65) (width 0.6) (layer "F.Cu") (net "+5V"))
 (segment (start 212.925 86.199316) (end 213.629316 85.495) (width 0.6) (layer "F.Cu") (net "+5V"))
 (segment (start 212.25 83.2075) (end 212.25 76.65) (width 0.6) (layer "F.Cu") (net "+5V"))
 (segment (start 196.3625 102.85) (end 198.65 105.1375) (width 0.6) (layer "F.Cu") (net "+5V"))
 (segment (start 214.5375 85.495) (end 212.25 83.2075) (width 0.6) (layer "F.Cu") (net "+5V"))
 (segment (start 213.629316 85.495) (end 214.5375 85.495) (width 0.6) (layer "F.Cu") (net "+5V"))
 (segment (start 198.65 105.1375) (end 202.1125 108.6) (width 0.6) (layer "F.Cu") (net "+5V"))
 (segment (start 200.65 100.95) (end 200.65 103.1375) (width 0.6) (layer "F.Cu") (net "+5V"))
 (segment (start 198.65 95.2) (end 198.65 100.95) (width 0.6) (layer "F.Cu") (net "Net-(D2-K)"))
 (segment (start 186.45 90.85) (end 194 90.85) (width 0.6) (layer "F.Cu") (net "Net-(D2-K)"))
 (segment (start 194.15 90.7) (end 198.65 95.2) (width 0.6) (layer "F.Cu") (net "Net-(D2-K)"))
 (segment (start 194 90.85) (end 194.15 90.7) (width 0.6) (layer "F.Cu") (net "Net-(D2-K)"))
 (segment (start 202.2 83.6) (end 202.2 82) (width 0.6) (layer "F.Cu") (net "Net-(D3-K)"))
 (segment (start 201.105804 74) (end 201.7 74.594196) (width 0.6) (layer "F.Cu") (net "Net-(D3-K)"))
 (segment (start 202.2 82) (end 201.7 81.5) (width 0.6) (layer "F.Cu") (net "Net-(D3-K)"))
 (segment (start 195 75.5) (end 196.5 74) (width 0.6) (layer "F.Cu") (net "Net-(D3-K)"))
 (segment (start 201.7 74.594196) (end 201.7 81.5) (width 0.6) (layer "F.Cu") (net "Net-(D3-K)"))
 (segment (start 201.7 81.5) (end 196.55 81.5) (width 0.6) (layer "F.Cu") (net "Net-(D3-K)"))
 (segment (start 196.5 74) (end 201.105804 74) (width 0.6) (layer "F.Cu") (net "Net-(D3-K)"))
 (segment (start 196.55 81.5) (end 189.2 88.85) (width 0.6) (layer "F.Cu") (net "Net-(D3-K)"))
 (segment (start 189.2 88.85) (end 186.45 88.85) (width 0.6) (layer "F.Cu") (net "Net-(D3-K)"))
 (segment (start 218.25 105.15) (end 219.05 105.95) (width 0.6) (layer "F.Cu") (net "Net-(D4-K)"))
 (segment (start 219.05 105.95) (end 219.05 106.65) (width 0.6) (layer "F.Cu") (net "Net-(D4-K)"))
 (segment (start 211.2 104) (end 212.958148 105.758148) (width 0.6) (layer "F.Cu") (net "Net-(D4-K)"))
 (segment (start 215.65 105.758148) (end 216.258148 105.15) (width 0.6) (layer "F.Cu") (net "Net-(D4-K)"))
 (segment (start 212.958148 105.758148) (end 215.65 105.758148) (width 0.6) (layer "F.Cu") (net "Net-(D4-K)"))
 (segment (start 216.258148 105.15) (end 218.25 105.15) (width 0.6) (layer "F.Cu") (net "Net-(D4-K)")))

